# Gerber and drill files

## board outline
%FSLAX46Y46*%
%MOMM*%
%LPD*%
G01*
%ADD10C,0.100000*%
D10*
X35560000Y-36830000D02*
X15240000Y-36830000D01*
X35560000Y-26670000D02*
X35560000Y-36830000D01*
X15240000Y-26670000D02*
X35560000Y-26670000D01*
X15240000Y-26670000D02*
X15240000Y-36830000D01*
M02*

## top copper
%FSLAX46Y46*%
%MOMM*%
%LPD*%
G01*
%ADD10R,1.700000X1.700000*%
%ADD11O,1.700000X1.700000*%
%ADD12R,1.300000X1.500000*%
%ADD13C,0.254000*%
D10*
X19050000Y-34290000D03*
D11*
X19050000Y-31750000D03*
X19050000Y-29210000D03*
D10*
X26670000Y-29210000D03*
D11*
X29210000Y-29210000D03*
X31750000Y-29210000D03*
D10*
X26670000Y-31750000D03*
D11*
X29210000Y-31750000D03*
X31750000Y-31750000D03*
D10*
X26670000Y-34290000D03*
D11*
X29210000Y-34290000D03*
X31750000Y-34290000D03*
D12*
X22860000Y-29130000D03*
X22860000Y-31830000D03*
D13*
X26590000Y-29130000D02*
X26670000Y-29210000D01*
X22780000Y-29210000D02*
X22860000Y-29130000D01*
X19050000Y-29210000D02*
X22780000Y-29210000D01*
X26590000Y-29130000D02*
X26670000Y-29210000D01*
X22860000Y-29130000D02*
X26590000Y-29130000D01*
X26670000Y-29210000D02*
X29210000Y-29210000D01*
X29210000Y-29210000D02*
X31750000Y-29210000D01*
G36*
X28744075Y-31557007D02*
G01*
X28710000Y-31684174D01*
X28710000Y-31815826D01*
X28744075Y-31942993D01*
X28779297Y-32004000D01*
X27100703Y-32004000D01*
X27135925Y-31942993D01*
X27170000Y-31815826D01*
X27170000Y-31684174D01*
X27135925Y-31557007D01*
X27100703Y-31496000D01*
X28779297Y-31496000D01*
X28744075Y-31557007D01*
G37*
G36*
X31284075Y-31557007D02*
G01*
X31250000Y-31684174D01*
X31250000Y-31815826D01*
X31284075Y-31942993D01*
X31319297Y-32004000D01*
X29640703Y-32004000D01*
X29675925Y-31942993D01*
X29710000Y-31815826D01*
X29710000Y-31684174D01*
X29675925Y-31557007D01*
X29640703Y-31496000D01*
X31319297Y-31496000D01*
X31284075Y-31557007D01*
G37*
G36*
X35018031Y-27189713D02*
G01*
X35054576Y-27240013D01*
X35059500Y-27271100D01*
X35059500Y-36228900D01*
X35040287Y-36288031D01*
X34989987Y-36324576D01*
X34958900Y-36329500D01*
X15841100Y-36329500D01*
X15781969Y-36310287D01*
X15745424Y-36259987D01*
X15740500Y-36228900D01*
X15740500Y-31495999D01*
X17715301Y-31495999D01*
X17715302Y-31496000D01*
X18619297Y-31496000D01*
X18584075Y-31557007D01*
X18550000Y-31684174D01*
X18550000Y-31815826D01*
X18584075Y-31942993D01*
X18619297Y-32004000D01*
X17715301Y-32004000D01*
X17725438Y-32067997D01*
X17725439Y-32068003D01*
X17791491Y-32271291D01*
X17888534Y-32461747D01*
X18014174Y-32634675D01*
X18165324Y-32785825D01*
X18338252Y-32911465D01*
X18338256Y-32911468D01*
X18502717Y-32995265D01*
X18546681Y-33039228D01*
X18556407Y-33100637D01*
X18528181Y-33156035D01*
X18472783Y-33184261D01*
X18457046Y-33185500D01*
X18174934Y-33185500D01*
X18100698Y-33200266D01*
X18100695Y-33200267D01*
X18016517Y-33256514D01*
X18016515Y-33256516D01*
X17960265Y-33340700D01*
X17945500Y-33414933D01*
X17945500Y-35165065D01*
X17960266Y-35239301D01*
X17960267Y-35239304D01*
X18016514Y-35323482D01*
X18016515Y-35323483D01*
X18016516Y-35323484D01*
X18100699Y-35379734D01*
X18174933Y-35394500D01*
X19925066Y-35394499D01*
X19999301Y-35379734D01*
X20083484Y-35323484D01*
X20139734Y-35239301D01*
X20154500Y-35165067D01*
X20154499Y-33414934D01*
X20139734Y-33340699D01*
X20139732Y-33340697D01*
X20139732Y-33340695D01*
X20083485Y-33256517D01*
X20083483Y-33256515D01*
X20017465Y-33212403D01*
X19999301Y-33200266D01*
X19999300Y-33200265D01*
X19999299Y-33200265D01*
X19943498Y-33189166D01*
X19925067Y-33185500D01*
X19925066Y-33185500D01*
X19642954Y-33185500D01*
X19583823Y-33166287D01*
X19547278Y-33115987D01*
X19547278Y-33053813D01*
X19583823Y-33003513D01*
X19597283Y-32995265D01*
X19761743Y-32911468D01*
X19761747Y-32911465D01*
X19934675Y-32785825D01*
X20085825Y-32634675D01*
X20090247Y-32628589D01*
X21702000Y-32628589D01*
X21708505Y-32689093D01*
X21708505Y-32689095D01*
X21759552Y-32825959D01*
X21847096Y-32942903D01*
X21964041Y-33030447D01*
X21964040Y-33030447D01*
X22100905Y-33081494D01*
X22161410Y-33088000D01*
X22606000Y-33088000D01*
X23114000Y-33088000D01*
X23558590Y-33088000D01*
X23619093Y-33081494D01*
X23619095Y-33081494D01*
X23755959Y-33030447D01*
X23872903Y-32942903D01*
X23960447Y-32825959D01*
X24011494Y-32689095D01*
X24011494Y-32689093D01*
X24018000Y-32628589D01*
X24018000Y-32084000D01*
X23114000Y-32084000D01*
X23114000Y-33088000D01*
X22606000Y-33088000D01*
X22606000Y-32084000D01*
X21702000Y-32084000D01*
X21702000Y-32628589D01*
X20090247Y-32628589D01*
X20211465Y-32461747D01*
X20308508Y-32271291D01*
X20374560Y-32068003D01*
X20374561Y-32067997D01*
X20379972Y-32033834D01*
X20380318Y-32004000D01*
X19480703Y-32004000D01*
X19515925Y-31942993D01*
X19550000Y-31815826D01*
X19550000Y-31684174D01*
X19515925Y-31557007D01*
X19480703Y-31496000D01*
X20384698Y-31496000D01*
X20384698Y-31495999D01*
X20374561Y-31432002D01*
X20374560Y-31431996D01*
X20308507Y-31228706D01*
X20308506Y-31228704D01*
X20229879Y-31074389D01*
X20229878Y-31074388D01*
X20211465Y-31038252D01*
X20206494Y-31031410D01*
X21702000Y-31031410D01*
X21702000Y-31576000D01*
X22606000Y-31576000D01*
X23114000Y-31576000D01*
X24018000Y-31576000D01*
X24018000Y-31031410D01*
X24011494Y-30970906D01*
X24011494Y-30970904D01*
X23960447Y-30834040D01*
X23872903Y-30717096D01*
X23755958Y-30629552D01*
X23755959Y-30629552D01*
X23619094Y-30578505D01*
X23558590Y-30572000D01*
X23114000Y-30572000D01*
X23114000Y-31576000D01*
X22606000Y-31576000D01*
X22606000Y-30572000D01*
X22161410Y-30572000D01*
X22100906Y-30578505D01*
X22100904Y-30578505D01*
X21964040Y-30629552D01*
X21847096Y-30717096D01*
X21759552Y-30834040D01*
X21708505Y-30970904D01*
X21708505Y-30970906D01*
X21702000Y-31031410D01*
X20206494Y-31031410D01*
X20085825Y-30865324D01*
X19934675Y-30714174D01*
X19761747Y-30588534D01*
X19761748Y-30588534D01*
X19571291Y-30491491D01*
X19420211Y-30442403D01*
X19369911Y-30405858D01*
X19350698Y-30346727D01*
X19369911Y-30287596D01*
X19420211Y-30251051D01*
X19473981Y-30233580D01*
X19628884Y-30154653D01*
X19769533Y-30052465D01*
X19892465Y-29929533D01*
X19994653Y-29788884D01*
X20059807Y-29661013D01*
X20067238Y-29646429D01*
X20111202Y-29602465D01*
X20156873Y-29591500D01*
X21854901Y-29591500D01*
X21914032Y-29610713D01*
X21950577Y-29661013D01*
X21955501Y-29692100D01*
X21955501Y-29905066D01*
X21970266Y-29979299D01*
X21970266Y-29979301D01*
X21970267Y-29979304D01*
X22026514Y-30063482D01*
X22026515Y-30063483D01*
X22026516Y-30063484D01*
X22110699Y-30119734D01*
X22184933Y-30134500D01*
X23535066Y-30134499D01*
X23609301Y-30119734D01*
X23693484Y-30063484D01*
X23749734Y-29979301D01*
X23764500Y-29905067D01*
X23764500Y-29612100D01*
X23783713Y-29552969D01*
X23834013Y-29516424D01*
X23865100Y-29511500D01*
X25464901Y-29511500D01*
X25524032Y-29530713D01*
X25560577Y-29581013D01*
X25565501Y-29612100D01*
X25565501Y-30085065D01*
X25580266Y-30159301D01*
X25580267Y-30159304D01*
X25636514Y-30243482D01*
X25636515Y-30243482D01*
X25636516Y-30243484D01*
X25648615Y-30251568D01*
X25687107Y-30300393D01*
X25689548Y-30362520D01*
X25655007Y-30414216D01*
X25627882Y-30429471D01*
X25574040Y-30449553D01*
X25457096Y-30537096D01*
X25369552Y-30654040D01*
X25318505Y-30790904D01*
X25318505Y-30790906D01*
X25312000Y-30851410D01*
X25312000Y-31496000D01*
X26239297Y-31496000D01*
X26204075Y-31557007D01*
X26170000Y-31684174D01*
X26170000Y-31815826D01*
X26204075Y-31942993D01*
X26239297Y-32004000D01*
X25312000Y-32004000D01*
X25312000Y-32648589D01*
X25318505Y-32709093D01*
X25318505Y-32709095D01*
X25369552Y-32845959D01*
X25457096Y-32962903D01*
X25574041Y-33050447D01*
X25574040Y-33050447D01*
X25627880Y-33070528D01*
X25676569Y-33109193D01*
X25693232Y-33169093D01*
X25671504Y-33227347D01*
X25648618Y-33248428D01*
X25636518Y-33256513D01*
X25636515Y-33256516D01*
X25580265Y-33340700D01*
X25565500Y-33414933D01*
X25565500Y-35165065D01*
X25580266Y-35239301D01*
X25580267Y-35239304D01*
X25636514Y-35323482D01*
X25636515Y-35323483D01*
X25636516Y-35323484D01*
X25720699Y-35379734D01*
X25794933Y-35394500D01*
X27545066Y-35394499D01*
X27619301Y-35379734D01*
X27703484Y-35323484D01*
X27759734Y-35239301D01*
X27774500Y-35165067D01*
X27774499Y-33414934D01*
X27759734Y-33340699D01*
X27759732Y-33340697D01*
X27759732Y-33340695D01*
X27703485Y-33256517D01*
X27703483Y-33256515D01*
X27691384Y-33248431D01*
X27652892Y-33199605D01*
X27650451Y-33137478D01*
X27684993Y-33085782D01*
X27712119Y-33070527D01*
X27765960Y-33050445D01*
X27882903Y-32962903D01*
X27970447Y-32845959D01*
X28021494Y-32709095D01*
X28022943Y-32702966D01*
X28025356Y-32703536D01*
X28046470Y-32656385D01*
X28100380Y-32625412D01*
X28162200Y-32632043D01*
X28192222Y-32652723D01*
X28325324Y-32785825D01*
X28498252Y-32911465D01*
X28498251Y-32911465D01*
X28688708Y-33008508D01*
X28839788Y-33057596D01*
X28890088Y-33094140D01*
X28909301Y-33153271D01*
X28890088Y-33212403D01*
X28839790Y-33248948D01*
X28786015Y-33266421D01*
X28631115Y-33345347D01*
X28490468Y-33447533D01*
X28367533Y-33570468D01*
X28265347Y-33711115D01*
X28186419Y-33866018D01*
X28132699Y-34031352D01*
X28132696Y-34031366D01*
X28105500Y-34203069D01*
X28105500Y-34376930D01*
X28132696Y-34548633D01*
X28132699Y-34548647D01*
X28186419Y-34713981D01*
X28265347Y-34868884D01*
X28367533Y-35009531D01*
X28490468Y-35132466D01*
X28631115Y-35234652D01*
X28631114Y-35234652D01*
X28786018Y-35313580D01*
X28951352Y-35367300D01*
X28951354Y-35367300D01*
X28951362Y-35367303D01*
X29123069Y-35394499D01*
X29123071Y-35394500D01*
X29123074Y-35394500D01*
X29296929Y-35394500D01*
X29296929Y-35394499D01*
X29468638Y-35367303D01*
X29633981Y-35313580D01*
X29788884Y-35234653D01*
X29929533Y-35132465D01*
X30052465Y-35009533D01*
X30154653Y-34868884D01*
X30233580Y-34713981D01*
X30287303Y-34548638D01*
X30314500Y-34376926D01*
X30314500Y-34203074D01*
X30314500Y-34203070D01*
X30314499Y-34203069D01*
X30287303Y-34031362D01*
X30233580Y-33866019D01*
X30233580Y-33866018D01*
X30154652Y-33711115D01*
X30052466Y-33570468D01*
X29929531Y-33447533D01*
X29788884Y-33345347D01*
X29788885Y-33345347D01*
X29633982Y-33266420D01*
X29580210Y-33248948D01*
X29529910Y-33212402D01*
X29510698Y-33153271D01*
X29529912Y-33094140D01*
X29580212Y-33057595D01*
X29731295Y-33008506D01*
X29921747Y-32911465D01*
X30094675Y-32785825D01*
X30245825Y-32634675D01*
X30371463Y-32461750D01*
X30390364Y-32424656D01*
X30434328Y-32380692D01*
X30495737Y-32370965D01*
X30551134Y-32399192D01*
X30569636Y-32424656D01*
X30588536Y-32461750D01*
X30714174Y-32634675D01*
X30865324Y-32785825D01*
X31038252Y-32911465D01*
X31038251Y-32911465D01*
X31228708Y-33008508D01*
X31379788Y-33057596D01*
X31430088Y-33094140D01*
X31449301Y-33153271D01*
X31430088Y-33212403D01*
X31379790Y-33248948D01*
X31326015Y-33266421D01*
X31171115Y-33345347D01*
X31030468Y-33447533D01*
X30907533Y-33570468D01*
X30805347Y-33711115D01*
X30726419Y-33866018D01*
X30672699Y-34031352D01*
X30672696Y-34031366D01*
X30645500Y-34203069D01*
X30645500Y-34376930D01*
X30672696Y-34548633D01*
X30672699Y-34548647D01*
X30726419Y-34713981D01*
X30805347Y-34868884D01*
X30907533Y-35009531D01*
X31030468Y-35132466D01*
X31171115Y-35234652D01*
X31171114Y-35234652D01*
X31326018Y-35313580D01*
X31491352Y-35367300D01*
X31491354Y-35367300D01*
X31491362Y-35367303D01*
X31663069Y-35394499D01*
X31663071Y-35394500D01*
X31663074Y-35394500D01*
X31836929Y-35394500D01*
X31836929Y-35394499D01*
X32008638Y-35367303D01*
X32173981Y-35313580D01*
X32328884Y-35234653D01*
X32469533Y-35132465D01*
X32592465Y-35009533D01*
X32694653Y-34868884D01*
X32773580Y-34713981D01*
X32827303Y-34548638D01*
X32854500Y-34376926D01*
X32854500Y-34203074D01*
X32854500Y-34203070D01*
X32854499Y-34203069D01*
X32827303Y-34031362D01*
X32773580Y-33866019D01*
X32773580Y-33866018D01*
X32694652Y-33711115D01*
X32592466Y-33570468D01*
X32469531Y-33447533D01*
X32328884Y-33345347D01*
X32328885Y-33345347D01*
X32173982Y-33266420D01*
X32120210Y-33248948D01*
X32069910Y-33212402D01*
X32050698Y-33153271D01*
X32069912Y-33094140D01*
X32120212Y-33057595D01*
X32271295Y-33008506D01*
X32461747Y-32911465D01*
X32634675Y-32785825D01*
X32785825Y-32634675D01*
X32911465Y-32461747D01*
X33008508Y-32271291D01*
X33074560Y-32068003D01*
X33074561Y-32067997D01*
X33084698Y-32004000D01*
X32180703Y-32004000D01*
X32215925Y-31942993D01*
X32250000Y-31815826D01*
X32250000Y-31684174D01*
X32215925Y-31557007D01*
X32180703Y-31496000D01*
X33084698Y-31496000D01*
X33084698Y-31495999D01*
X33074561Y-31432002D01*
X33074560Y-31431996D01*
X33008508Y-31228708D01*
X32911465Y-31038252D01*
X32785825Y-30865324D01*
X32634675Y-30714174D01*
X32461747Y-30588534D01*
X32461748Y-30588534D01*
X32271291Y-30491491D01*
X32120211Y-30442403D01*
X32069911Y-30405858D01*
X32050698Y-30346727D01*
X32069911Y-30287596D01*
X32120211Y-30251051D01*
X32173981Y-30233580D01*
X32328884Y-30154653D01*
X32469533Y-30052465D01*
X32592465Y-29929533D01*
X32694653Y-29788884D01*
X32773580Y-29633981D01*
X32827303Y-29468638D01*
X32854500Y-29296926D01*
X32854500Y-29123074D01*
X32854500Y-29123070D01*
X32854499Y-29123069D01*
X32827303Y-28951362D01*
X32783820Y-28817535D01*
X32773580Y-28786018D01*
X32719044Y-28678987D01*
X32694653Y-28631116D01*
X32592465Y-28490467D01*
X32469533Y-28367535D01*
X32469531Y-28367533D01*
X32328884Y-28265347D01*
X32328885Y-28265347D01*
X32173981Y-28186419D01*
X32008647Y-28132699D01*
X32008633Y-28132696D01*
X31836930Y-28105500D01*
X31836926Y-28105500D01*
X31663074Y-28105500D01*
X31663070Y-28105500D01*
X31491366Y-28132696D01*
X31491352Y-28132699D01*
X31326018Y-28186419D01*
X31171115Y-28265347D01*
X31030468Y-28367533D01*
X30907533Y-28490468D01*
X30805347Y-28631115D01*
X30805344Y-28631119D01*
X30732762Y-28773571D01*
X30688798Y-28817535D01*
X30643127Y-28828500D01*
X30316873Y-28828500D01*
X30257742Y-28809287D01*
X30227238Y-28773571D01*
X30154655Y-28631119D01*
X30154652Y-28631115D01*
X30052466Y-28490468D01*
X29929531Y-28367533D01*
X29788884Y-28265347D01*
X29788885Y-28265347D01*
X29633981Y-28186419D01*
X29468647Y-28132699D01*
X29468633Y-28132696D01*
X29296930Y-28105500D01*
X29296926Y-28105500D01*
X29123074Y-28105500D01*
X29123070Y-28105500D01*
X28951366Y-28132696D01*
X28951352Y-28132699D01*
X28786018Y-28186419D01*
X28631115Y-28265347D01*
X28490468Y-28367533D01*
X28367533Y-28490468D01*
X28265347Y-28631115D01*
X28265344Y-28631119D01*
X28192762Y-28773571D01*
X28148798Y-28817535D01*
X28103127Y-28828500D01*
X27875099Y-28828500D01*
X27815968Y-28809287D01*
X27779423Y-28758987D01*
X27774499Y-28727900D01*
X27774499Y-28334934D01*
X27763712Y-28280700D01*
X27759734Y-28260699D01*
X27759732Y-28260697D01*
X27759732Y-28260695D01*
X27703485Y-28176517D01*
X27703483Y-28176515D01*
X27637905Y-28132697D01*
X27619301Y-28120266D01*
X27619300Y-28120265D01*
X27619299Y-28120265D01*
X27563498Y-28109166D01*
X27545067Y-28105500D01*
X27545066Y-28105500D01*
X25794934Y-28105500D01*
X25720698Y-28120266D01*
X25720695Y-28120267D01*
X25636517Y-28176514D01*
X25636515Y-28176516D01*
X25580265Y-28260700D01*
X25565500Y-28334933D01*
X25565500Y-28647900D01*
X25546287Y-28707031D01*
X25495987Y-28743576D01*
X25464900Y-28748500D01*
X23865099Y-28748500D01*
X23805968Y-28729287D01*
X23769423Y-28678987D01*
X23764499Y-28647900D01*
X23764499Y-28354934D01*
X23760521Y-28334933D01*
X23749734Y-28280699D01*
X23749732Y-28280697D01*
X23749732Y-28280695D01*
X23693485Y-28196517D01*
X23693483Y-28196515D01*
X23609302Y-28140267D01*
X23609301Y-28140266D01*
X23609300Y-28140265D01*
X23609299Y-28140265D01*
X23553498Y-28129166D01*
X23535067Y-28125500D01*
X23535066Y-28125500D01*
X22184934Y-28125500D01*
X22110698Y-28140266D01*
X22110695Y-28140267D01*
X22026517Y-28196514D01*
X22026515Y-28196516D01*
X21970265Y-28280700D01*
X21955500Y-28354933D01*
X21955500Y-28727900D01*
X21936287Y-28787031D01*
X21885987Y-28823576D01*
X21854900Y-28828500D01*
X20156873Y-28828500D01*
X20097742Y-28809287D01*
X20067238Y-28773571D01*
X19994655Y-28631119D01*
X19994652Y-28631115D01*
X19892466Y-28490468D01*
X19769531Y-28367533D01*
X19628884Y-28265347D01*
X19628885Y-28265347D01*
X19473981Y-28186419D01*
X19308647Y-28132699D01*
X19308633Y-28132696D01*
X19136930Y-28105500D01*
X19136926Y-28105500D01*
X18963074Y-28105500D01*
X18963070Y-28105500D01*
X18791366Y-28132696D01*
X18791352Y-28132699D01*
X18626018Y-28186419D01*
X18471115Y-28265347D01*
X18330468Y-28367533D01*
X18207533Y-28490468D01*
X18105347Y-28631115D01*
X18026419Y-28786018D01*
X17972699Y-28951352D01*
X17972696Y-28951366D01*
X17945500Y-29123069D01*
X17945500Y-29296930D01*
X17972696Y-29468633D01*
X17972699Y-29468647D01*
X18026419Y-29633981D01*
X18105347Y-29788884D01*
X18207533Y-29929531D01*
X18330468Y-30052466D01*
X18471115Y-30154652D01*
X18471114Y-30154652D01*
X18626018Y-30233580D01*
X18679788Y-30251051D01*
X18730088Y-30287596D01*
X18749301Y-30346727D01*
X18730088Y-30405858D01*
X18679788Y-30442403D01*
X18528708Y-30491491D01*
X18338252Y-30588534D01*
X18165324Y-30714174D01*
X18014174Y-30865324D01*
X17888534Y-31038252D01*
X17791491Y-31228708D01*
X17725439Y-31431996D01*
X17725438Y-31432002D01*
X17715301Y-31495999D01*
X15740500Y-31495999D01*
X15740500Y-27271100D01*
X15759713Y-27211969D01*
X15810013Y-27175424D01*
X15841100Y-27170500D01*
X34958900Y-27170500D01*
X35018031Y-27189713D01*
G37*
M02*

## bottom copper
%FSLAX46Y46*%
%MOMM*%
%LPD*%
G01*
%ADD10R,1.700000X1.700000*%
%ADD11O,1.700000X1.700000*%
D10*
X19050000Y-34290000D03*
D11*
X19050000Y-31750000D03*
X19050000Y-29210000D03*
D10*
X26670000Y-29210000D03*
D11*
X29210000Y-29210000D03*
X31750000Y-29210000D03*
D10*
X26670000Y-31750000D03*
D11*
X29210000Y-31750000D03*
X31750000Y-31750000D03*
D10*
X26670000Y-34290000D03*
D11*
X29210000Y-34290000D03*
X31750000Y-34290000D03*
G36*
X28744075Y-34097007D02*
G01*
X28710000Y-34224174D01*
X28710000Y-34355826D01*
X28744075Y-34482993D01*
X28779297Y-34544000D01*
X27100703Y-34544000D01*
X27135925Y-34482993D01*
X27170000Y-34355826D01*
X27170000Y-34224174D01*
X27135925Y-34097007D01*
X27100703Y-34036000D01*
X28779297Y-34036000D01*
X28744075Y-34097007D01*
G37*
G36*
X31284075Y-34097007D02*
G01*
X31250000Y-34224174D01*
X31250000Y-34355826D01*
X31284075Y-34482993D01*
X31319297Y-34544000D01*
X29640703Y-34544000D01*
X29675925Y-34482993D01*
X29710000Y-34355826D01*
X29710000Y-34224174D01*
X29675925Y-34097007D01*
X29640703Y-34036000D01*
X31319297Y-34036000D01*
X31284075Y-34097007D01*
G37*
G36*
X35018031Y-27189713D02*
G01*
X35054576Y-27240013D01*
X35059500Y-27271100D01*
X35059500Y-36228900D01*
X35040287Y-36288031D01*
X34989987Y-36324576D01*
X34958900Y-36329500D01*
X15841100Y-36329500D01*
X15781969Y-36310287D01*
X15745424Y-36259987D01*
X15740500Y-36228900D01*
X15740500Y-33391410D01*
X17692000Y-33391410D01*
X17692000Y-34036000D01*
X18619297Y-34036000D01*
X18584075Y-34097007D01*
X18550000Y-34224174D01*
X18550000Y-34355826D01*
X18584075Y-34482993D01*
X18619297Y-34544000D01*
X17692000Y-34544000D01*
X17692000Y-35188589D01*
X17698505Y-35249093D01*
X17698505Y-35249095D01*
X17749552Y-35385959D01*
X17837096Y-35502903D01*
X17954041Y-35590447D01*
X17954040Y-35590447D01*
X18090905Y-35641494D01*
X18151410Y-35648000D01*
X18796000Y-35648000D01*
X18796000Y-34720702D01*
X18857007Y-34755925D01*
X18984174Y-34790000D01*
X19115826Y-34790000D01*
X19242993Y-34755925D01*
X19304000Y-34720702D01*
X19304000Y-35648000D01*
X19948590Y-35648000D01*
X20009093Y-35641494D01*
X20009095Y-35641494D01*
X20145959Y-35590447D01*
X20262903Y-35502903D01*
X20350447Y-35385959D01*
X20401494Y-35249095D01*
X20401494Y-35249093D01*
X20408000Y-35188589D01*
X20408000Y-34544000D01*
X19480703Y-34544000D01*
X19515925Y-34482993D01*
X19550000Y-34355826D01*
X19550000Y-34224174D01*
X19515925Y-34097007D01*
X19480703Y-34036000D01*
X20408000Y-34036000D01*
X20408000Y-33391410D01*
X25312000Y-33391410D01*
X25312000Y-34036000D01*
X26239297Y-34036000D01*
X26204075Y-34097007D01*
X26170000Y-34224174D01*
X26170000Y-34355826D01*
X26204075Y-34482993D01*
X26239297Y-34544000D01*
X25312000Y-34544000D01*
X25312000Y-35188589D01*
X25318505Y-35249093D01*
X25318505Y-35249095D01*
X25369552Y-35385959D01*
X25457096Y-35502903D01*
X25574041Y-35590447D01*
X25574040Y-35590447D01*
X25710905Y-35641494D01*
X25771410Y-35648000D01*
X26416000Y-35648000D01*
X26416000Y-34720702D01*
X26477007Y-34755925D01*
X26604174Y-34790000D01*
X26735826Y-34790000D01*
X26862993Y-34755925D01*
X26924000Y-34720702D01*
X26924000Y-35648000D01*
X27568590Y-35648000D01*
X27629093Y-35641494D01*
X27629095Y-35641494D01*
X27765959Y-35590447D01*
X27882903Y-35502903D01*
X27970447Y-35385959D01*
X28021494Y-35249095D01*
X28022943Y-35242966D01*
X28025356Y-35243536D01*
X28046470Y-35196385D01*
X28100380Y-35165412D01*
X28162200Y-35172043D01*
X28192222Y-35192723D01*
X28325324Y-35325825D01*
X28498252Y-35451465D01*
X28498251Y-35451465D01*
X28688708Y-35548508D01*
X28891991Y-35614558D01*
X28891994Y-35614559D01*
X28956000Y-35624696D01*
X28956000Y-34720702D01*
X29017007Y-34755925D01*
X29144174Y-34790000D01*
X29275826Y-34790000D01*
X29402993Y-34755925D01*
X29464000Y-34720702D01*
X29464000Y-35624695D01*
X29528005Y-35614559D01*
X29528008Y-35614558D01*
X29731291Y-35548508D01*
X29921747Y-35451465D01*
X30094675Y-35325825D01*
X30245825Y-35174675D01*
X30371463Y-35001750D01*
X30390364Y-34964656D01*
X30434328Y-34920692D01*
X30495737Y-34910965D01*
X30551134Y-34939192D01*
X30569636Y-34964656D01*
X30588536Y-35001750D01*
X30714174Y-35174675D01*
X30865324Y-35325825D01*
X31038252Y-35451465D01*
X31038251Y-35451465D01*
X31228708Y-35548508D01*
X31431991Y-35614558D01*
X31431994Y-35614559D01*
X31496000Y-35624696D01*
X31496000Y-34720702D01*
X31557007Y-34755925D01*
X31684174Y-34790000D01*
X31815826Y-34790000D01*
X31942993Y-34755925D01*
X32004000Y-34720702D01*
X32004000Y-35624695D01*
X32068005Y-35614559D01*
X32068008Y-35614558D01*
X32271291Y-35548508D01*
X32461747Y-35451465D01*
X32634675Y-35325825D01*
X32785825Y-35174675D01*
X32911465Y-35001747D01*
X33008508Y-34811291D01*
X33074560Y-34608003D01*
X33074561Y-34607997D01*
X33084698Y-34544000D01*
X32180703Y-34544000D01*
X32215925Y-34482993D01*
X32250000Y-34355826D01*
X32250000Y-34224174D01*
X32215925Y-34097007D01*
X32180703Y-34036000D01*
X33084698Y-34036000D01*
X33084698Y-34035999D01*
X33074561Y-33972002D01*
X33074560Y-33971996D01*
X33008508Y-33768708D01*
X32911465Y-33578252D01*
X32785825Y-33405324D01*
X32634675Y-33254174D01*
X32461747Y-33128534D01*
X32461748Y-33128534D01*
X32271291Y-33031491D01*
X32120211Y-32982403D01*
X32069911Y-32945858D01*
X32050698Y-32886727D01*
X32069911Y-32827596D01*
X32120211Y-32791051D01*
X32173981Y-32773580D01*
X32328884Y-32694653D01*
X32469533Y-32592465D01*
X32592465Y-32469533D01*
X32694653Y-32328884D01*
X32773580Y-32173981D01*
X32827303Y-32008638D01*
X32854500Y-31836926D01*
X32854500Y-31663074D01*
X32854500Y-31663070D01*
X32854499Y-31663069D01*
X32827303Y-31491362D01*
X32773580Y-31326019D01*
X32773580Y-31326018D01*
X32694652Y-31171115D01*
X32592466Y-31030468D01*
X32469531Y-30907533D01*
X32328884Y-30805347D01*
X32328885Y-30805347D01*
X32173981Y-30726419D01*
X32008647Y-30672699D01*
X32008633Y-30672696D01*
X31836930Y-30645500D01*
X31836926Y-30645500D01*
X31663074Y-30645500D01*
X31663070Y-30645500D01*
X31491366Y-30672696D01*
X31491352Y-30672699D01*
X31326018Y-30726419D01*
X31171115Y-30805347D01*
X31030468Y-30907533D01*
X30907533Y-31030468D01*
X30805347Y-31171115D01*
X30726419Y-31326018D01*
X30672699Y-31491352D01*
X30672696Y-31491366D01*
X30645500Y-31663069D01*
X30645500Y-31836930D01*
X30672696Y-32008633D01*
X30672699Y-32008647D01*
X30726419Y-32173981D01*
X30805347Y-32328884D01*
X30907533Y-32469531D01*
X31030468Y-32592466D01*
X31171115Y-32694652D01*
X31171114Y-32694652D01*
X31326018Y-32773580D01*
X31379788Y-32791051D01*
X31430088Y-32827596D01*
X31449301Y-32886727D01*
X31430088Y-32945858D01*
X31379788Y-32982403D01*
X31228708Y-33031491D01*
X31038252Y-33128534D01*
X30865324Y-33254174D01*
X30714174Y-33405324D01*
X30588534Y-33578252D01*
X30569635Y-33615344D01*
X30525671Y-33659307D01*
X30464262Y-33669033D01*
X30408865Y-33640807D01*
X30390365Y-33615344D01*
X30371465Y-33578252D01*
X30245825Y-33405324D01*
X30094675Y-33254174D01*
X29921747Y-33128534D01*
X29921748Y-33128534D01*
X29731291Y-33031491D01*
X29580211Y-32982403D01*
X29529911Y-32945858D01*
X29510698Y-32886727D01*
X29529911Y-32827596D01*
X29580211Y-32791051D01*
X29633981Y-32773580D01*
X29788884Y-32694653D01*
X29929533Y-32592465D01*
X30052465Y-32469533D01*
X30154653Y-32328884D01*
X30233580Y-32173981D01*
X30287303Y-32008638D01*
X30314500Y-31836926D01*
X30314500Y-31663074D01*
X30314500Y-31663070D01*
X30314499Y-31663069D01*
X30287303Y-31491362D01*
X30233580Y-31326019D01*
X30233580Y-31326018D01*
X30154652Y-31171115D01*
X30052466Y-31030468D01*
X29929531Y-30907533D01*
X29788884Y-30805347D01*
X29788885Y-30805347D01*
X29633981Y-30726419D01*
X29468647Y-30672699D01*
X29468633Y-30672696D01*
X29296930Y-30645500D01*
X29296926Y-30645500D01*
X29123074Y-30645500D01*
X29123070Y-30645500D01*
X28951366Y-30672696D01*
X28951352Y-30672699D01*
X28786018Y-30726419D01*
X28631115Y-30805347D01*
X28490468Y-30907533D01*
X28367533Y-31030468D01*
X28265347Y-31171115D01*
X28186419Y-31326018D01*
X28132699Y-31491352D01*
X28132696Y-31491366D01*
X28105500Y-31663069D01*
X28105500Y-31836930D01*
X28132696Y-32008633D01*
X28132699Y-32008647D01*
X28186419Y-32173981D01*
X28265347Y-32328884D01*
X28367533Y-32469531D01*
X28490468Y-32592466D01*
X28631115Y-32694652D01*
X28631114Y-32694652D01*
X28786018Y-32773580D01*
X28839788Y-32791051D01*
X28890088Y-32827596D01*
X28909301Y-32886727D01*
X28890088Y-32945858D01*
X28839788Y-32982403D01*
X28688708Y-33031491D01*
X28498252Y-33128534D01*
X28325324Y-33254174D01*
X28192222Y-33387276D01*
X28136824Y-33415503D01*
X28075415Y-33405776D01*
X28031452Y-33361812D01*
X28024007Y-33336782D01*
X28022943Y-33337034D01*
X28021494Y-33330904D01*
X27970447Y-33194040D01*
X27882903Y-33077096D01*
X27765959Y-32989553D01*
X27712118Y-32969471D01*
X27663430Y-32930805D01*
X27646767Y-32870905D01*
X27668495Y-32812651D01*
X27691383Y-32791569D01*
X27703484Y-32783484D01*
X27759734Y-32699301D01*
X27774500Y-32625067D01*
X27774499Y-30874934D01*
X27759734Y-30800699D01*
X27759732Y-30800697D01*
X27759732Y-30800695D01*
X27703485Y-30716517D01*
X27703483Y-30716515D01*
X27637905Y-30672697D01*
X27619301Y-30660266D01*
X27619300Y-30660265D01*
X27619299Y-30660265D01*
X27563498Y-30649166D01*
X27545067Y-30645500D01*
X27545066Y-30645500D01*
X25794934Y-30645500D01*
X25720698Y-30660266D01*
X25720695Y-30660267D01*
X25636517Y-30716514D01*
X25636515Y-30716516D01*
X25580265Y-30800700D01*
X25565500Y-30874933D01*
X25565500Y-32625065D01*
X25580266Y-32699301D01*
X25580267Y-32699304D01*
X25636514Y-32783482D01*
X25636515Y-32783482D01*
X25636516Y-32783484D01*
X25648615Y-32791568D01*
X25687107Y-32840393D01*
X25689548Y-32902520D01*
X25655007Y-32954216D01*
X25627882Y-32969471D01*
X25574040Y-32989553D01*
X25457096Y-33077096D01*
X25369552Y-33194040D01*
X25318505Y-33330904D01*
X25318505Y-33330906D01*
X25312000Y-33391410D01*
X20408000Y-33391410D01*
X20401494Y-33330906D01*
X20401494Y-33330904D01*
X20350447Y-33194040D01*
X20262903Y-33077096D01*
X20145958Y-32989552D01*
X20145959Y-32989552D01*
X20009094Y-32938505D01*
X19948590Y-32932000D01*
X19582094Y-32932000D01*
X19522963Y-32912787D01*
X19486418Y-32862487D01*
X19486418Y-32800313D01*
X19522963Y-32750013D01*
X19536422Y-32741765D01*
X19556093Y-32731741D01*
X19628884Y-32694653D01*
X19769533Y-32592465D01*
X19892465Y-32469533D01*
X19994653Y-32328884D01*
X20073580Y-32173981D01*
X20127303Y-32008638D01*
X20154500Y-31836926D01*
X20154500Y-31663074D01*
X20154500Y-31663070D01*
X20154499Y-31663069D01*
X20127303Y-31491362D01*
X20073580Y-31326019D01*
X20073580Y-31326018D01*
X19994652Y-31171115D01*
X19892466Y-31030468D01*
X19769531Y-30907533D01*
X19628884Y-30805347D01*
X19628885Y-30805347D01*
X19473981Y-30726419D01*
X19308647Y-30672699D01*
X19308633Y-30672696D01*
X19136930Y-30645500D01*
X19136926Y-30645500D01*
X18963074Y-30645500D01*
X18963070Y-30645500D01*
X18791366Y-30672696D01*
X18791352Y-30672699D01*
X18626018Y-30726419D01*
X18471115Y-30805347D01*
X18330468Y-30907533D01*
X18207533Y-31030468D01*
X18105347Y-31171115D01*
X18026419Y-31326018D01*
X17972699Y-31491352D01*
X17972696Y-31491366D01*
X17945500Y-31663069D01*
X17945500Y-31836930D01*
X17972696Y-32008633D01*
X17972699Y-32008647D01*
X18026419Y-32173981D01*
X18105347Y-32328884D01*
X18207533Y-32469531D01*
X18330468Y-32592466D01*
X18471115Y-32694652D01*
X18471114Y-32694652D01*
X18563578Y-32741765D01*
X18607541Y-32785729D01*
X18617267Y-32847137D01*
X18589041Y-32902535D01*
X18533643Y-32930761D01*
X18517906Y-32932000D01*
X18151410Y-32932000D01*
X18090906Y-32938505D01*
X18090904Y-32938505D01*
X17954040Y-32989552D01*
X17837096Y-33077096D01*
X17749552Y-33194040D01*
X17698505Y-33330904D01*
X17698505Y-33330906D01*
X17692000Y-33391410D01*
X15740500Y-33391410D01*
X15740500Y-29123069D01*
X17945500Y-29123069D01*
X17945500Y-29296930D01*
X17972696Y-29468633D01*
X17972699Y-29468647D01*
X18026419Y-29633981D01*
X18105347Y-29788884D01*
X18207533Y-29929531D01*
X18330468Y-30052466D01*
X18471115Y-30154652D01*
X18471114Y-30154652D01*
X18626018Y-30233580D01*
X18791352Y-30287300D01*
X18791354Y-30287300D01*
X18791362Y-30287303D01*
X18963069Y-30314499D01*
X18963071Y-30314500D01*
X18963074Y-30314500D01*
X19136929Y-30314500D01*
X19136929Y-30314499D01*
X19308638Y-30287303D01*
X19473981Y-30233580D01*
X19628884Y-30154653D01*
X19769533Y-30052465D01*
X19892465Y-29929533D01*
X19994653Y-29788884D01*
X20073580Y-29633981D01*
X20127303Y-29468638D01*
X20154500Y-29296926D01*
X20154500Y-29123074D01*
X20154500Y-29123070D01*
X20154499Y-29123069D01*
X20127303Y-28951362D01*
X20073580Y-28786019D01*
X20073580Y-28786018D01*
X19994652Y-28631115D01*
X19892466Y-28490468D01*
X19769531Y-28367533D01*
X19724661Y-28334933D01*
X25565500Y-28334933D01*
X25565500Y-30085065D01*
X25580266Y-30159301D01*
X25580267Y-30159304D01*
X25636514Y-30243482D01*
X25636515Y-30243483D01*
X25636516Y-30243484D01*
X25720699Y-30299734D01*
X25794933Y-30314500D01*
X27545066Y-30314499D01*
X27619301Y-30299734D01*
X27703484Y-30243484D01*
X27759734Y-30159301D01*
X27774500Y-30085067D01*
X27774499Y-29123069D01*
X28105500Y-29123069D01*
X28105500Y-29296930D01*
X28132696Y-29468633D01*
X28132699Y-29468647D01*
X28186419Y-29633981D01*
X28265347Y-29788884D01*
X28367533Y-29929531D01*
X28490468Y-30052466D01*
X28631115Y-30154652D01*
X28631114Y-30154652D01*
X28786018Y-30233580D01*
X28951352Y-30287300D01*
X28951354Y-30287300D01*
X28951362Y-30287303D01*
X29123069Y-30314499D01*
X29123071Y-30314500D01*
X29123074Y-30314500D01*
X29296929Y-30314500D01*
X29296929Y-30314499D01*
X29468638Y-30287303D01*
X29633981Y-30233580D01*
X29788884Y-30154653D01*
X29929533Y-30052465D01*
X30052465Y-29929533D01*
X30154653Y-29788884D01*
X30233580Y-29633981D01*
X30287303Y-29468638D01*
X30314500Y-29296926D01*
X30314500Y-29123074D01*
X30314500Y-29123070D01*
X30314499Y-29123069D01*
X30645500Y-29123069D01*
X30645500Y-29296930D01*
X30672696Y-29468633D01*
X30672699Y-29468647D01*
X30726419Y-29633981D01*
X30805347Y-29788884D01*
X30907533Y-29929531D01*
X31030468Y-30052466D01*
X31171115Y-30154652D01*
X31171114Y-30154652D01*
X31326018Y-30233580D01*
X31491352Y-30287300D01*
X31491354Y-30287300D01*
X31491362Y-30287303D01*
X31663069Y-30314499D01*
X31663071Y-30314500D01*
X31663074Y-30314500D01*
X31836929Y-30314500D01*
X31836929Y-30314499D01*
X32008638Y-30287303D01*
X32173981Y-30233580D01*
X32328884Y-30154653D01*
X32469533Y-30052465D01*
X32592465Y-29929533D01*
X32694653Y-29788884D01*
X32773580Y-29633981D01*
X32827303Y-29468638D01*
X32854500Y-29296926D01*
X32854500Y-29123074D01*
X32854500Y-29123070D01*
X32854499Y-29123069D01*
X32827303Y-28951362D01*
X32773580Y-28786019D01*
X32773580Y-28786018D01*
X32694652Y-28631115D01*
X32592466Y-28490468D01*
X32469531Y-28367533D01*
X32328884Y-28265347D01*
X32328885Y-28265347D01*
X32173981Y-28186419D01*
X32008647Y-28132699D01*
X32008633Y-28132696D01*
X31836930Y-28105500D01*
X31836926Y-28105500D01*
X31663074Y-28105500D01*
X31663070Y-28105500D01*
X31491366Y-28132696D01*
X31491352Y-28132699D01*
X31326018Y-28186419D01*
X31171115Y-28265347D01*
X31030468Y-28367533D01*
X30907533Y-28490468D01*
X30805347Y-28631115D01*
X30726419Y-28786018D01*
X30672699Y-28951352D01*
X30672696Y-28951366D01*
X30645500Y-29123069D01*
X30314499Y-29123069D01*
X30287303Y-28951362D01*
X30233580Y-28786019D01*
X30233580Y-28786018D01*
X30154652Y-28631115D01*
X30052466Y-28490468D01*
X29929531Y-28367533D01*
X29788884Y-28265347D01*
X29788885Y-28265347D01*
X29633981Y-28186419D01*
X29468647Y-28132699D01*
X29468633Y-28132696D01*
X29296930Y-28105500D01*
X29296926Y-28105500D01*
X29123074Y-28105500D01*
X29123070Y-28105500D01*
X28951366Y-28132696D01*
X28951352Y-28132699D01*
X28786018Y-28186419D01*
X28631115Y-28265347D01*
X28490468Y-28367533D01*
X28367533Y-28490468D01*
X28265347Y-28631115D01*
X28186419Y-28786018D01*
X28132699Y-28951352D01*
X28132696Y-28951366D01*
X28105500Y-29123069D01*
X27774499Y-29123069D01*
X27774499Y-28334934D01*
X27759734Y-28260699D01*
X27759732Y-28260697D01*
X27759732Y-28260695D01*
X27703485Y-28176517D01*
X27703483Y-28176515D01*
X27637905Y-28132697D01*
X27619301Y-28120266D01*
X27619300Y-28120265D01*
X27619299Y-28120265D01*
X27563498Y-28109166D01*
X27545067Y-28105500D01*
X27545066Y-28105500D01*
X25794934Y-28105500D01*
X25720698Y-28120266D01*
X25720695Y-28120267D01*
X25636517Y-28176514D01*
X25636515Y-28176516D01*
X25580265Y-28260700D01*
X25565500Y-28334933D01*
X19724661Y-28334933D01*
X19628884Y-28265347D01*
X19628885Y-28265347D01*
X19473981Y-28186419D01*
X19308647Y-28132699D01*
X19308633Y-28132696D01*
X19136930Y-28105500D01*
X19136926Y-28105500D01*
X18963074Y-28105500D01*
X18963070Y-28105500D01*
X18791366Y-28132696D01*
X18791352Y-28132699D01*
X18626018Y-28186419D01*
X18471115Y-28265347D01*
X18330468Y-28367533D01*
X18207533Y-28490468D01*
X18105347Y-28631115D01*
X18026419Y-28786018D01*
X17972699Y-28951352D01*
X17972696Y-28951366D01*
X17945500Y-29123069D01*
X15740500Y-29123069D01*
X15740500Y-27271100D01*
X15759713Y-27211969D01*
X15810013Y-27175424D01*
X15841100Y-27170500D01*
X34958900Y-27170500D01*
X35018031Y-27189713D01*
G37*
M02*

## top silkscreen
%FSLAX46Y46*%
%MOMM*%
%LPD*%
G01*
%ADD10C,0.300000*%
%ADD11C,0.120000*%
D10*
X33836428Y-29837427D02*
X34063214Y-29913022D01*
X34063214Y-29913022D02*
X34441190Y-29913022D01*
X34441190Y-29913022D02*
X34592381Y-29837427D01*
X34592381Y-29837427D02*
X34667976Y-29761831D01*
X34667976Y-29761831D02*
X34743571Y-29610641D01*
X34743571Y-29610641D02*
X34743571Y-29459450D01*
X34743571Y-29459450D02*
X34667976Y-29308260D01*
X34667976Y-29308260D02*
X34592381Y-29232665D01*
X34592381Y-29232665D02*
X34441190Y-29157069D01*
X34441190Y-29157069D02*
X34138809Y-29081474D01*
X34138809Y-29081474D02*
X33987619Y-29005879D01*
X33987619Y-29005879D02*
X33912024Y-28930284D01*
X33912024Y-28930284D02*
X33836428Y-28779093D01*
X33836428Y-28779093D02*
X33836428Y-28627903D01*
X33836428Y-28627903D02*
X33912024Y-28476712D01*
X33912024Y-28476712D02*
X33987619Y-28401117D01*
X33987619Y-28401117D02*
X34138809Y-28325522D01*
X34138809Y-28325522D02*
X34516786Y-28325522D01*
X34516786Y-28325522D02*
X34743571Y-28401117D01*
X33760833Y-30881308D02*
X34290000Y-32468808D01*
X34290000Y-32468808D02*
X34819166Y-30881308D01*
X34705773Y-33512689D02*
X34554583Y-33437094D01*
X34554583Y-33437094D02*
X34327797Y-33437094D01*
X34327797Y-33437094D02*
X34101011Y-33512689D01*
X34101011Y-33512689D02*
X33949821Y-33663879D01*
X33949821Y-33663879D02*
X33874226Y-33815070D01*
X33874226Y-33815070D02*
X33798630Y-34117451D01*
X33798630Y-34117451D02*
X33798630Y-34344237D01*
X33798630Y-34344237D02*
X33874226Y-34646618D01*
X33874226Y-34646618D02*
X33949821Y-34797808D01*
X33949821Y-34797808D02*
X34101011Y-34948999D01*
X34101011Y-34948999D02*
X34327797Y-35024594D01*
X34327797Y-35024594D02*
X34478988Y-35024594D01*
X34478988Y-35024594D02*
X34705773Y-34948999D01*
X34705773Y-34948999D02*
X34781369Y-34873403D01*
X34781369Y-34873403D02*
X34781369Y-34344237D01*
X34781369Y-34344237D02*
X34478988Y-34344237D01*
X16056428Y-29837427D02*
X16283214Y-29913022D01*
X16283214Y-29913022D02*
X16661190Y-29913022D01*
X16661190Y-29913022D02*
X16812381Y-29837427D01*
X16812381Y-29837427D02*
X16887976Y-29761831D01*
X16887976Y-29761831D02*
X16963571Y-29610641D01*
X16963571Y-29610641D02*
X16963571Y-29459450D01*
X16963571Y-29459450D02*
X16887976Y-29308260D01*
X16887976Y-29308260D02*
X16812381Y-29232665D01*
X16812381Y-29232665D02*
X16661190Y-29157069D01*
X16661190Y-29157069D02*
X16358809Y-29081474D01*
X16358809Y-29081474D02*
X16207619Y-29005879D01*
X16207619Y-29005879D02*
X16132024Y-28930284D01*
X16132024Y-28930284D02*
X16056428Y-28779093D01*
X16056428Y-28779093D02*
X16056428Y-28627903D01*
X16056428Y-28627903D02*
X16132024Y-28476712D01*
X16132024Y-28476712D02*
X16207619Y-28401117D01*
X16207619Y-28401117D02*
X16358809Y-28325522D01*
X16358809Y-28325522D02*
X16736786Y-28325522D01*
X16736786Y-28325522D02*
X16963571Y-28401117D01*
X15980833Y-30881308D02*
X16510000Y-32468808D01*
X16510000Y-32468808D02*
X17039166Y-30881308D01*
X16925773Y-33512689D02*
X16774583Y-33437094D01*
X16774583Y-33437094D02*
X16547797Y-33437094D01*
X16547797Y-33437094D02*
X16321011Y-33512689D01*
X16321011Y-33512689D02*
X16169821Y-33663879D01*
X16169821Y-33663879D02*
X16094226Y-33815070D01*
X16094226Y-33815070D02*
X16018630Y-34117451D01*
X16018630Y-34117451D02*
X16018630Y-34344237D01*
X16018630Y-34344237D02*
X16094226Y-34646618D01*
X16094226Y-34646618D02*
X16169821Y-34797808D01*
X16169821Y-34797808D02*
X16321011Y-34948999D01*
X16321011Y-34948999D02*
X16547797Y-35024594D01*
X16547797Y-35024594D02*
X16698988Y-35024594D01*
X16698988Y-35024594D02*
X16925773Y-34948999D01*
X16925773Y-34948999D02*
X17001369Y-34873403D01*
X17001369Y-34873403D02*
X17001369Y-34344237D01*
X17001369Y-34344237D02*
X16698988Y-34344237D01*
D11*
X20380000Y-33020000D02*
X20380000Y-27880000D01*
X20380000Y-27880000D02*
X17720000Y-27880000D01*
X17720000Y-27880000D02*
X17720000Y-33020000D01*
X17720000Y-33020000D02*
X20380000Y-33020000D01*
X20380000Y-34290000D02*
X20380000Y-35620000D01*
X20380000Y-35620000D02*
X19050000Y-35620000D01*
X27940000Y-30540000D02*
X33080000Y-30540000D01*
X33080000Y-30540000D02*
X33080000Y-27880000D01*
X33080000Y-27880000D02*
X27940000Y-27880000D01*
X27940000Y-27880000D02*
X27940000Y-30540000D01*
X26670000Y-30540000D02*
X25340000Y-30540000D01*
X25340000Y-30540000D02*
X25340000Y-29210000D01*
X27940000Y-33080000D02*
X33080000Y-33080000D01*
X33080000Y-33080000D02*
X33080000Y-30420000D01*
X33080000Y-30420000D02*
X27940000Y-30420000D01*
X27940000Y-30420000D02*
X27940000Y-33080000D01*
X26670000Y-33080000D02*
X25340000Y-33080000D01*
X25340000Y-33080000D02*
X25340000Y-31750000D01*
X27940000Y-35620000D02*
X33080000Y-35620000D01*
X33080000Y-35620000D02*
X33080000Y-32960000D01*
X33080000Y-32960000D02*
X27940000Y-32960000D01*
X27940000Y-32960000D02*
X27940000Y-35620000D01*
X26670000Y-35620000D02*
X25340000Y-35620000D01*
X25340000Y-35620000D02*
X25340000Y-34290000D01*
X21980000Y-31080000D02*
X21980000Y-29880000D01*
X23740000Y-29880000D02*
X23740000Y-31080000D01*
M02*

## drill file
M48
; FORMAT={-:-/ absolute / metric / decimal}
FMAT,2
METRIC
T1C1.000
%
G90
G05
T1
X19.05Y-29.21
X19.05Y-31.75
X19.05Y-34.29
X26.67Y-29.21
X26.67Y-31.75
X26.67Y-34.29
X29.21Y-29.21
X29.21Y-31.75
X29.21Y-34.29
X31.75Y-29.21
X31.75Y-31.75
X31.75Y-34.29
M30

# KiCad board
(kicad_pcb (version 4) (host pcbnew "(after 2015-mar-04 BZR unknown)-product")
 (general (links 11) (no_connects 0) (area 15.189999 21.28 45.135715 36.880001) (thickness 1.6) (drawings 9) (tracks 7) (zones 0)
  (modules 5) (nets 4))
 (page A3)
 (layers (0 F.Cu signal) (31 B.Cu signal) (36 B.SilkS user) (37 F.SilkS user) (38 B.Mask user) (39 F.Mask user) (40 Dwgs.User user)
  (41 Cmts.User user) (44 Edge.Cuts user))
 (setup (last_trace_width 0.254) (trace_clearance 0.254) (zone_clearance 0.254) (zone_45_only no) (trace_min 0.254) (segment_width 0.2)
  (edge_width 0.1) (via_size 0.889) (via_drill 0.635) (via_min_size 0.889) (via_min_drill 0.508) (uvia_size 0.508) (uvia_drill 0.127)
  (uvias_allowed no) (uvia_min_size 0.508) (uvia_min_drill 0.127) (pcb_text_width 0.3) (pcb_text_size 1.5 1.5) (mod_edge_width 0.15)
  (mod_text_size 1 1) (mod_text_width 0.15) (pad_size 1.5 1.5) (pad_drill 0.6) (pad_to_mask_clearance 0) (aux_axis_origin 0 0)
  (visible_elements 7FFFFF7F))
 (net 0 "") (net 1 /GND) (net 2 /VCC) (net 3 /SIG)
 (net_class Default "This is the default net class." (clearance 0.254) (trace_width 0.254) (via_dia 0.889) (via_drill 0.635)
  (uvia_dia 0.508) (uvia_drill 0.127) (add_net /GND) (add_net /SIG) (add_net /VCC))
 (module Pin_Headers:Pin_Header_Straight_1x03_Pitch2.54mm (layer F.Cu) (at 19.05 34.29 180)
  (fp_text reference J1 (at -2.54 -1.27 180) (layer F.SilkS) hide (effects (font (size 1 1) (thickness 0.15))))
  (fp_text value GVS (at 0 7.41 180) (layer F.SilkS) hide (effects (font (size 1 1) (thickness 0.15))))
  (fp_line (start -1.33 1.27) (end -1.33 6.41) (layer F.SilkS) (width 0.12))
  (fp_line (start -1.33 6.41) (end 1.33 6.41) (layer F.SilkS) (width 0.12))
  (fp_line (start 1.33 6.41) (end 1.33 1.27) (layer F.SilkS) (width 0.12))
  (fp_line (start 1.33 1.27) (end -1.33 1.27) (layer F.SilkS) (width 0.12))
  (fp_line (start -1.33 0) (end -1.33 -1.33) (layer F.SilkS) (width 0.12))
  (fp_line (start -1.33 -1.33) (end 0 -1.33) (layer F.SilkS) (width 0.12))
  (pad 1 thru_hole rect (at 0 0 180) (size 1.7 1.7) (drill 1) (layers *.Cu *.Mask) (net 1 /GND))
  (pad 2 thru_hole oval (at 0 2.54 180) (size 1.7 1.7) (drill 1) (layers *.Cu *.Mask) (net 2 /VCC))
  (pad 3 thru_hole oval (at 0 5.08 180) (size 1.7 1.7) (drill 1) (layers *.Cu *.Mask) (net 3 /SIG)))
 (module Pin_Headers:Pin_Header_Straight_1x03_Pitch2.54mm (layer F.Cu) (at 26.67 29.21 90)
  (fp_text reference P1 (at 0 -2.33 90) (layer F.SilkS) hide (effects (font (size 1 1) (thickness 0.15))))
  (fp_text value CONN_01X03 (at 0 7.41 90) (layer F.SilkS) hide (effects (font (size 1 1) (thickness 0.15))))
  (fp_line (start -1.33 1.27) (end -1.33 6.41) (layer F.SilkS) (width 0.12))
  (fp_line (start -1.33 6.41) (end 1.33 6.41) (layer F.SilkS) (width 0.12))
  (fp_line (start 1.33 6.41) (end 1.33 1.27) (layer F.SilkS) (width 0.12))
  (fp_line (start 1.33 1.27) (end -1.33 1.27) (layer F.SilkS) (width 0.12))
  (fp_line (start -1.33 0) (end -1.33 -1.33) (layer F.SilkS) (width 0.12))
  (fp_line (start -1.33 -1.33) (end 0 -1.33) (layer F.SilkS) (width 0.12))
  (pad 1 thru_hole rect (at 0 0 90) (size 1.7 1.7) (drill 1) (layers *.Cu *.Mask) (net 3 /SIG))
  (pad 2 thru_hole oval (at 0 2.54 90) (size 1.7 1.7) (drill 1) (layers *.Cu *.Mask) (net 3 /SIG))
  (pad 3 thru_hole oval (at 0 5.08 90) (size 1.7 1.7) (drill 1) (layers *.Cu *.Mask) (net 3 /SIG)))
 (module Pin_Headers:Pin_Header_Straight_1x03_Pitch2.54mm (layer F.Cu) (at 26.67 31.75 90)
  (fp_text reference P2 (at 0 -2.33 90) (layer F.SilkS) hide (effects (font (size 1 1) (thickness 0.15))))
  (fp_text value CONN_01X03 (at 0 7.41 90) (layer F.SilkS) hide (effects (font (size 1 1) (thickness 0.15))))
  (fp_line (start -1.33 1.27) (end -1.33 6.41) (layer F.SilkS) (width 0.12))
  (fp_line (start -1.33 6.41) (end 1.33 6.41) (layer F.SilkS) (width 0.12))
  (fp_line (start 1.33 6.41) (end 1.33 1.27) (layer F.SilkS) (width 0.12))
  (fp_line (start 1.33 1.27) (end -1.33 1.27) (layer F.SilkS) (width 0.12))
  (fp_line (start -1.33 0) (end -1.33 -1.33) (layer F.SilkS) (width 0.12))
  (fp_line (start -1.33 -1.33) (end 0 -1.33) (layer F.SilkS) (width 0.12))
  (pad 1 thru_hole rect (at 0 0 90) (size 1.7 1.7) (drill 1) (layers *.Cu *.Mask) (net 2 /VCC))
  (pad 2 thru_hole oval (at 0 2.54 90) (size 1.7 1.7) (drill 1) (layers *.Cu *.Mask) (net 2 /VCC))
  (pad 3 thru_hole oval (at 0 5.08 90) (size 1.7 1.7) (drill 1) (layers *.Cu *.Mask) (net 2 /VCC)))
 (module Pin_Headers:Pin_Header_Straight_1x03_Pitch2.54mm (layer F.Cu) (at 26.67 34.29 90)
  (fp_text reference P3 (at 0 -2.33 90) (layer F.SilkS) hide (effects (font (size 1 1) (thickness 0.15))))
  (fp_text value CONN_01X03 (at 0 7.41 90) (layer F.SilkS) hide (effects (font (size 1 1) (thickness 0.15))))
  (fp_line (start -1.33 1.27) (end -1.33 6.41) (layer F.SilkS) (width 0.12))
  (fp_line (start -1.33 6.41) (end 1.33 6.41) (layer F.SilkS) (width 0.12))
  (fp_line (start 1.33 6.41) (end 1.33 1.27) (layer F.SilkS) (width 0.12))
  (fp_line (start 1.33 1.27) (end -1.33 1.27) (layer F.SilkS) (width 0.12))
  (fp_line (start -1.33 0) (end -1.33 -1.33) (layer F.SilkS) (width 0.12))
  (fp_line (start -1.33 -1.33) (end 0 -1.33) (layer F.SilkS) (width 0.12))
  (pad 1 thru_hole rect (at 0 0 90) (size 1.7 1.7) (drill 1) (layers *.Cu *.Mask) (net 1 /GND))
  (pad 2 thru_hole oval (at 0 2.54 90) (size 1.7 1.7) (drill 1) (layers *.Cu *.Mask) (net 1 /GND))
  (pad 3 thru_hole oval (at 0 5.08 90) (size 1.7 1.7) (drill 1) (layers *.Cu *.Mask) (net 1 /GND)))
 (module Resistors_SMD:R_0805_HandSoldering (layer F.Cu) (at 22.86 30.48 270)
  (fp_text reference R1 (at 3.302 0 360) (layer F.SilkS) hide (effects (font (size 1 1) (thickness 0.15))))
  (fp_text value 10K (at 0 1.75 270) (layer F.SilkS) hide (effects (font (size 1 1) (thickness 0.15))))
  (fp_line (start 0.6 0.88) (end -0.6 0.88) (layer F.SilkS) (width 0.12))
  (fp_line (start -0.6 -0.88) (end 0.6 -0.88) (layer F.SilkS) (width 0.12))
  (pad 1 smd rect (at -1.35 0 270) (size 1.5 1.3) (layers F.Cu F.Mask) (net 3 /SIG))
  (pad 2 smd rect (at 1.35 0 270) (size 1.5 1.3) (layers F.Cu F.Mask) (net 2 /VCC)))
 (gr_line (start 35.56 36.83) (end 15.24 36.83) (angle 90) (layer Edge.Cuts) (width 0.1))
 (gr_line (start 35.56 26.67) (end 35.56 36.83) (angle 90) (layer Edge.Cuts) (width 0.1))
 (gr_line (start 15.24 26.67) (end 35.56 26.67) (angle 90) (layer Edge.Cuts) (width 0.1))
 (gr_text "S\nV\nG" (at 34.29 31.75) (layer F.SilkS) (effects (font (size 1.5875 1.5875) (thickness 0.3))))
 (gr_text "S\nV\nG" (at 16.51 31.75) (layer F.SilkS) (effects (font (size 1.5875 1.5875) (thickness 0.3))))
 (gr_line (start 15.24 26.67) (end 15.24 36.83) (angle 90) (layer Edge.Cuts) (width 0.1))
 (segment (start 26.59 29.13) (end 26.67 29.21) (width 0.254) (layer F.Cu) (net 3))
 (segment (start 22.78 29.21) (end 22.86 29.13) (width 0.254) (layer F.Cu) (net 3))
 (segment (start 19.05 29.21) (end 22.78 29.21) (width 0.254) (layer F.Cu) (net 3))
 (segment (start 26.59 29.13) (end 26.67 29.21) (width 0.254) (layer F.Cu) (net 3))
 (segment (start 22.86 29.13) (end 26.59 29.13) (width 0.254) (layer F.Cu) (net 3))
 (segment (start 26.67 29.21) (end 29.21 29.21) (width 0.254) (layer F.Cu) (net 3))
 (segment (start 29.21 29.21) (end 31.75 29.21) (width 0.254) (layer F.Cu) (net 3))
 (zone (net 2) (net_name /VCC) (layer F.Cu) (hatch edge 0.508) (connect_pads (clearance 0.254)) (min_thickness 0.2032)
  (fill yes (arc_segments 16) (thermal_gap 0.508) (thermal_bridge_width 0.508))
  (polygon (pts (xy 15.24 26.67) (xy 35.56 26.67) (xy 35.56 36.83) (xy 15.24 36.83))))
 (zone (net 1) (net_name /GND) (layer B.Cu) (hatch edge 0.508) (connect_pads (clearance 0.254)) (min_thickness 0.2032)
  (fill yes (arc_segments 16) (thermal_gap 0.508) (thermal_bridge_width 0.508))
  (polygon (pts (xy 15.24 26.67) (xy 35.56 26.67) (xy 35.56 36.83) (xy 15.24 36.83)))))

